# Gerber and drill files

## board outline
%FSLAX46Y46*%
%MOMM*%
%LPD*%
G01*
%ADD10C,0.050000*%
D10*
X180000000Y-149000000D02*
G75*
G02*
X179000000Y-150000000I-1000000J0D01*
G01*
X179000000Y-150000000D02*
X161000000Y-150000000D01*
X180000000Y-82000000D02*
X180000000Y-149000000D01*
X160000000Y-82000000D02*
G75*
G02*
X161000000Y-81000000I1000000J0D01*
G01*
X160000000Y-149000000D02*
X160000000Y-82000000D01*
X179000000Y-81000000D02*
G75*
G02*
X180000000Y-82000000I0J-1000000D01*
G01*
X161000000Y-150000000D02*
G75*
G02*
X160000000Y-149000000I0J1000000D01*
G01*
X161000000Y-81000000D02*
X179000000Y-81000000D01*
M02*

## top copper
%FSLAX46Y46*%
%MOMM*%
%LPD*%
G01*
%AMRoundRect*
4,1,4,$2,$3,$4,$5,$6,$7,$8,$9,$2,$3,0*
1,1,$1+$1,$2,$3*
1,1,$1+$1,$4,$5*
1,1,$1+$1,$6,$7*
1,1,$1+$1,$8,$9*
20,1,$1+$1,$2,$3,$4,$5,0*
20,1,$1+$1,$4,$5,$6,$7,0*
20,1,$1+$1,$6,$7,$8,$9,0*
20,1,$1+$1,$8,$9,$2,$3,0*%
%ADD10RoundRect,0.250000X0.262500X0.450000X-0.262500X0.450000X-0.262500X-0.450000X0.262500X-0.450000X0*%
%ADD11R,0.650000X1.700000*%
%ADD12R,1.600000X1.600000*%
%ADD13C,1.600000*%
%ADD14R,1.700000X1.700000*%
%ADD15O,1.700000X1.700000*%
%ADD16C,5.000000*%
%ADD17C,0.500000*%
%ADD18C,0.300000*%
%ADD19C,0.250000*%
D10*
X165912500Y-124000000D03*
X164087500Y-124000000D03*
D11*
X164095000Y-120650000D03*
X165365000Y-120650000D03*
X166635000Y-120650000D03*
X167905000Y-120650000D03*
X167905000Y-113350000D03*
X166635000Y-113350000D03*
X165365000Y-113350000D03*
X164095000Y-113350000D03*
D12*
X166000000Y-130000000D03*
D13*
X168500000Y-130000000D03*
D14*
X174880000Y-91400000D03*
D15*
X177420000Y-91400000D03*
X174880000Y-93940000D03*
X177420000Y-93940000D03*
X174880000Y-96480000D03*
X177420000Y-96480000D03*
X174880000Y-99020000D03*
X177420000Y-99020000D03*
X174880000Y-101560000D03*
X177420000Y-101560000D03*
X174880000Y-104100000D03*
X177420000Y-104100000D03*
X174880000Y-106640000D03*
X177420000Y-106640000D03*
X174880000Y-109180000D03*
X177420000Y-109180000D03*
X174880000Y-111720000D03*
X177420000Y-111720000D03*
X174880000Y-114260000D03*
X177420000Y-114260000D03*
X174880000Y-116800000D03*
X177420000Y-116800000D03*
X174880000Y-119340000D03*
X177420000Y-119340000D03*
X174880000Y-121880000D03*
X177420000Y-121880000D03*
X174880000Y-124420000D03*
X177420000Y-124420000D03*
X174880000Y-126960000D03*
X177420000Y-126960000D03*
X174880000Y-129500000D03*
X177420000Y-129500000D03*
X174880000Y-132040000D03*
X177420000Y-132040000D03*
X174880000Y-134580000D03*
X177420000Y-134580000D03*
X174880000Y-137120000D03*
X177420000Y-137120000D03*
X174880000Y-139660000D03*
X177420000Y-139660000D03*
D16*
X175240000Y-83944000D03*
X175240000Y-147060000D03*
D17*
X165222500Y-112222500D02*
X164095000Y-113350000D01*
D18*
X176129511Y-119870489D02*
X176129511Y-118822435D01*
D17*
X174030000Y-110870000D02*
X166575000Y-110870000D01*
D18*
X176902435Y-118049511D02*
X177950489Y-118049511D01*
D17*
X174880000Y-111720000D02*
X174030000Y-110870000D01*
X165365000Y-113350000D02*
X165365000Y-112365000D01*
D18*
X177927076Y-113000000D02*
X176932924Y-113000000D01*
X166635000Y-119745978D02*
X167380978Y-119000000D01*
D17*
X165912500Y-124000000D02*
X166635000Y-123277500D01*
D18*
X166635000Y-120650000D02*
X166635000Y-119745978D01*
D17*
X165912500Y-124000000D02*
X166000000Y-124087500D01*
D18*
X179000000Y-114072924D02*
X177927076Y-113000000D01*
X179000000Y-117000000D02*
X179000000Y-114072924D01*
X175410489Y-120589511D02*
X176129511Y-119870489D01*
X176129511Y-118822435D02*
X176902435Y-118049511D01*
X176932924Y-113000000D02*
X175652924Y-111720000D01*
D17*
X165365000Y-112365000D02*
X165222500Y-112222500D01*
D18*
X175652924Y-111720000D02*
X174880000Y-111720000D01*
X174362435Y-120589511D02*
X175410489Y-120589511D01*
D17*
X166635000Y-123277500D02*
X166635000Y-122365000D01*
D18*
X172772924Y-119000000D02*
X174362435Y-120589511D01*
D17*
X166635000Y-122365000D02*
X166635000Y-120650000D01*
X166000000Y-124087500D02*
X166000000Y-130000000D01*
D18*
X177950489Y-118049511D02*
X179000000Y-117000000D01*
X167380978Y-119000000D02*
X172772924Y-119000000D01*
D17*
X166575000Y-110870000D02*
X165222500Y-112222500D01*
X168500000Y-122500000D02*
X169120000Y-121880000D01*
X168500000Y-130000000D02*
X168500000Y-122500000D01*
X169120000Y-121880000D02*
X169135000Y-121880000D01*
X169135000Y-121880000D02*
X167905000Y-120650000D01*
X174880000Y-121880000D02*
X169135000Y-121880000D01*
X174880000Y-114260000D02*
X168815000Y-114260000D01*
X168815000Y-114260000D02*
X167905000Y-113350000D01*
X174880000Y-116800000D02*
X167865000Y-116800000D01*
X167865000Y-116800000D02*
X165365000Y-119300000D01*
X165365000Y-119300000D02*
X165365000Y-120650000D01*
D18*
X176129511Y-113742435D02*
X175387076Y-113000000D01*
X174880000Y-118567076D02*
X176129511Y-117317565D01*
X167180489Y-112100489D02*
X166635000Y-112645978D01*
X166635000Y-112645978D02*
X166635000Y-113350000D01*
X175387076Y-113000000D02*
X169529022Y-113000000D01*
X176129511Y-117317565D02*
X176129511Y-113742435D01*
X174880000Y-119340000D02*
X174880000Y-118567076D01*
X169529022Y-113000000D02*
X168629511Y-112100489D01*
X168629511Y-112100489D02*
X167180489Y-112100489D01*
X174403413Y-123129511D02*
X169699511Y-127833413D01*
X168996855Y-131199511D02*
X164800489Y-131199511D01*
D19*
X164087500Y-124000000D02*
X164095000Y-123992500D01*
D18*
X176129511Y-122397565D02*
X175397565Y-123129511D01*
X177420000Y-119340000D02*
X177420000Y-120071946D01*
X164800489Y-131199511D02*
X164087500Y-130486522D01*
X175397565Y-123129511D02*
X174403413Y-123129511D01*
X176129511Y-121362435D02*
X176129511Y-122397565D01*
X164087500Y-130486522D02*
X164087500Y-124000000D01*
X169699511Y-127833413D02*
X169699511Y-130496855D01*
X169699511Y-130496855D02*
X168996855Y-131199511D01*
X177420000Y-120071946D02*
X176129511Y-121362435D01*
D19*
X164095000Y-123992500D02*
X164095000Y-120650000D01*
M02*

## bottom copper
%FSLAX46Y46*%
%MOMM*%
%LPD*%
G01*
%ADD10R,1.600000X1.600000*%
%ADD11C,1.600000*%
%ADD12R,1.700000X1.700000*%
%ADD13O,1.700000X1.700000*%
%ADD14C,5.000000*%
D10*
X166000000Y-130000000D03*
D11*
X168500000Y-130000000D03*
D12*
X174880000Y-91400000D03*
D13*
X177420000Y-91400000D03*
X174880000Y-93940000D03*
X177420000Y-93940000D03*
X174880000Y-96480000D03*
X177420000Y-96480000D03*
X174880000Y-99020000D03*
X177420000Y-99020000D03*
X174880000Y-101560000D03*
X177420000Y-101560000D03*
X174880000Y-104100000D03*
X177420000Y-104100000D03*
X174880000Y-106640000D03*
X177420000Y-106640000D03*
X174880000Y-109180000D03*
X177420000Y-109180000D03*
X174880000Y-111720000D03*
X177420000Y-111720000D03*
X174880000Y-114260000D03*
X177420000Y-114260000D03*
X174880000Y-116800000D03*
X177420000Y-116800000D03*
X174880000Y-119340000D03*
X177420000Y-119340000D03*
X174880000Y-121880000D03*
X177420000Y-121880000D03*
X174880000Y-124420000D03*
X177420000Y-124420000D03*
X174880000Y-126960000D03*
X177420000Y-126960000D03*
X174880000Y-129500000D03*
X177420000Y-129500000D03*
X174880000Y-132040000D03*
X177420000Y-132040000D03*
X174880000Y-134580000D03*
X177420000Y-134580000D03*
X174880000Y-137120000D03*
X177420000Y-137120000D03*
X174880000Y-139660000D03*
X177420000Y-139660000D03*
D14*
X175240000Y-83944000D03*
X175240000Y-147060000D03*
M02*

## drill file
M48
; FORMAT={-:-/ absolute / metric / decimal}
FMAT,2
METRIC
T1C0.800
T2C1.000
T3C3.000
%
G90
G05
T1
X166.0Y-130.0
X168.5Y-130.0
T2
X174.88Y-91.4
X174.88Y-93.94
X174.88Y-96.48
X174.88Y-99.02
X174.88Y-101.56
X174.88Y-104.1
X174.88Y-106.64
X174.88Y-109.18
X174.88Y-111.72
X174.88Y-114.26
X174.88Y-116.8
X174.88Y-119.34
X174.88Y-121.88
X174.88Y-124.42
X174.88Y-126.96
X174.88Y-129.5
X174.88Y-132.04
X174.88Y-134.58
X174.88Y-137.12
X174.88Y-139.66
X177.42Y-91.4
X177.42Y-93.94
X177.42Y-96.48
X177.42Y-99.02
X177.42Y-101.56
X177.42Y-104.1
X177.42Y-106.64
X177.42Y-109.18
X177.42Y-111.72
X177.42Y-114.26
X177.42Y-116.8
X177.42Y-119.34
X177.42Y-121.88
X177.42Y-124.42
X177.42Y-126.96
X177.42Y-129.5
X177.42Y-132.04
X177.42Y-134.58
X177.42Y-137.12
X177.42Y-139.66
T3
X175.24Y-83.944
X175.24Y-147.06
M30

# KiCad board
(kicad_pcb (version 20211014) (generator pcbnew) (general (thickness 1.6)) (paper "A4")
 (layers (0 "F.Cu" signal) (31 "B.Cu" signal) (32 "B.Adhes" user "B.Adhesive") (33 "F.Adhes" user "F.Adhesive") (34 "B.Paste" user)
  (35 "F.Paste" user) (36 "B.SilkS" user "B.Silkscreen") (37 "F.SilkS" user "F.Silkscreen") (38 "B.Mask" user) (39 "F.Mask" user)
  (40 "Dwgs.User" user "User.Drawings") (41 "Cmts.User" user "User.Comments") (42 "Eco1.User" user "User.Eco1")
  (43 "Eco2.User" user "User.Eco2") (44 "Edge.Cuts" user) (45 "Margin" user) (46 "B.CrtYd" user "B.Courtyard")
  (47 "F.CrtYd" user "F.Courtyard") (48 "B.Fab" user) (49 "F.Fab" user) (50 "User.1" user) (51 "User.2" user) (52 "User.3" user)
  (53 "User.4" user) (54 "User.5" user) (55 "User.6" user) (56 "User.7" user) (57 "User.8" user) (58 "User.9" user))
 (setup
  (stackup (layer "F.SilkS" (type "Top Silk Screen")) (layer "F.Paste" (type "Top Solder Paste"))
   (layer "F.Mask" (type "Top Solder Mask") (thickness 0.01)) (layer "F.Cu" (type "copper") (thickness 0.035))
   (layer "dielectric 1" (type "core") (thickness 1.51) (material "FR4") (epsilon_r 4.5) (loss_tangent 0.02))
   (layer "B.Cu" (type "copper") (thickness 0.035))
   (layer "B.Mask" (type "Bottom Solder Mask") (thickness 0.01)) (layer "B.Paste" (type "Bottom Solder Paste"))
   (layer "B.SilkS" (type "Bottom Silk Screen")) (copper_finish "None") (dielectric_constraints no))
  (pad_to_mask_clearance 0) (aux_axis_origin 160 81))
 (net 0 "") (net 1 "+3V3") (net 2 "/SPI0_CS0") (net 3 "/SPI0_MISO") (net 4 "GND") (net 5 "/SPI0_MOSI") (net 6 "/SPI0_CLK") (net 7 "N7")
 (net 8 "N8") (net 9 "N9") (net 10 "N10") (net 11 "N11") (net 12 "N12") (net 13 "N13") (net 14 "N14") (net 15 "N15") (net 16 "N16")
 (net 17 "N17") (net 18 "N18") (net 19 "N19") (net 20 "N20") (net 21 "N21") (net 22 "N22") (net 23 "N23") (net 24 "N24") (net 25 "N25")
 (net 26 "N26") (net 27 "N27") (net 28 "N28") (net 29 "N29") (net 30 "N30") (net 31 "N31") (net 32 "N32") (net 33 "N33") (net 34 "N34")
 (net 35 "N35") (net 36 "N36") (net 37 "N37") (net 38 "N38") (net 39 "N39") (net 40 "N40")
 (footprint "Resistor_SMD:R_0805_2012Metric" (layer "F.Cu") (at 165 124 180)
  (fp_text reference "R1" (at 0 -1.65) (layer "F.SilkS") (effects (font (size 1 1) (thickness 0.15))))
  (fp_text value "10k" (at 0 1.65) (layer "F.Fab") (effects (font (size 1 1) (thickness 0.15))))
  (pad "1" smd roundrect (at -0.9125 0 180) (size 1.025 1.4) (layers "F.Cu" "F.Paste" "F.Mask") (roundrect_rratio 0.243902439)
   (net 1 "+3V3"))
  (pad "2" smd roundrect (at 0.9125 0 180) (size 1.025 1.4) (layers "F.Cu" "F.Paste" "F.Mask") (roundrect_rratio 0.243902439)
   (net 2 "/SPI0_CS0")))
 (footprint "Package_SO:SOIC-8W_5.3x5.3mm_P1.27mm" (layer "F.Cu") (at 166 117 90)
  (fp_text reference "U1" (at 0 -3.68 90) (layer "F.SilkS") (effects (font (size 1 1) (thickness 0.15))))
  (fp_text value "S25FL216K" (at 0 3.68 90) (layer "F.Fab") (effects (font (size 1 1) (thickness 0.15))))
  (pad "1" smd rect (at -3.65 -1.905 90) (size 1.7 0.65) (layers "F.Cu" "F.Paste" "F.Mask") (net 2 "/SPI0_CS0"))
  (pad "2" smd rect (at -3.65 -0.635 90) (size 1.7 0.65) (layers "F.Cu" "F.Paste" "F.Mask") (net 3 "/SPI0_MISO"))
  (pad "3" smd rect (at -3.65 0.635 90) (size 1.7 0.65) (layers "F.Cu" "F.Paste" "F.Mask") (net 1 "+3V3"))
  (pad "4" smd rect (at -3.65 1.905 90) (size 1.7 0.65) (layers "F.Cu" "F.Paste" "F.Mask") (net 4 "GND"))
  (pad "5" smd rect (at 3.65 1.905 90) (size 1.7 0.65) (layers "F.Cu" "F.Paste" "F.Mask") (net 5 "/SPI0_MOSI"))
  (pad "6" smd rect (at 3.65 0.635 90) (size 1.7 0.65) (layers "F.Cu" "F.Paste" "F.Mask") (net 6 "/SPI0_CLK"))
  (pad "7" smd rect (at 3.65 -0.635 90) (size 1.7 0.65) (layers "F.Cu" "F.Paste" "F.Mask") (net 1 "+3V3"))
  (pad "8" smd rect (at 3.65 -1.905 90) (size 1.7 0.65) (layers "F.Cu" "F.Paste" "F.Mask") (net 1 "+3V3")))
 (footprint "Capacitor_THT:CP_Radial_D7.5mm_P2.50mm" (layer "F.Cu") (at 166 130)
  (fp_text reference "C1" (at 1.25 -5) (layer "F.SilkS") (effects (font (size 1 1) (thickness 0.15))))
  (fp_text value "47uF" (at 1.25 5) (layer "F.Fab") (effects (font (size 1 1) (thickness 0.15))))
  (pad "1" thru_hole rect (at 0 0) (size 1.6 1.6) (drill 0.8) (layers *.Cu *.Mask) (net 1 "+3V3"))
  (pad "2" thru_hole circle (at 2.5 0) (size 1.6 1.6) (drill 0.8) (layers *.Cu *.Mask) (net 4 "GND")))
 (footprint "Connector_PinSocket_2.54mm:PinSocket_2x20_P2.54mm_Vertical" (layer "B.Cu") (at 174.88 91.4 180)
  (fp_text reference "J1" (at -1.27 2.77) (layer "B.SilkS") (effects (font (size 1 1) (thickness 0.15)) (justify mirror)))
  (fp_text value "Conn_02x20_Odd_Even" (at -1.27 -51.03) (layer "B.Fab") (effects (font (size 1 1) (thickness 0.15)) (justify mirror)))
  (pad "1" thru_hole rect (at 0 0 180) (size 1.7 1.7) (drill 1) (layers *.Cu *.Mask) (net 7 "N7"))
  (pad "2" thru_hole oval (at -2.54 0 180) (size 1.7 1.7) (drill 1) (layers *.Cu *.Mask) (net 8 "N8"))
  (pad "3" thru_hole oval (at 0 -2.54 180) (size 1.7 1.7) (drill 1) (layers *.Cu *.Mask) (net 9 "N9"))
  (pad "4" thru_hole oval (at -2.54 -2.54 180) (size 1.7 1.7) (drill 1) (layers *.Cu *.Mask) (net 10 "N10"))
  (pad "5" thru_hole oval (at 0 -5.08 180) (size 1.7 1.7) (drill 1) (layers *.Cu *.Mask) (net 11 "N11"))
  (pad "6" thru_hole oval (at -2.54 -5.08 180) (size 1.7 1.7) (drill 1) (layers *.Cu *.Mask) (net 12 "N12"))
  (pad "7" thru_hole oval (at 0 -7.62 180) (size 1.7 1.7) (drill 1) (layers *.Cu *.Mask) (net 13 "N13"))
  (pad "8" thru_hole oval (at -2.54 -7.62 180) (size 1.7 1.7) (drill 1) (layers *.Cu *.Mask) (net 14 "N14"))
  (pad "9" thru_hole oval (at 0 -10.16 180) (size 1.7 1.7) (drill 1) (layers *.Cu *.Mask) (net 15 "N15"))
  (pad "10" thru_hole oval (at -2.54 -10.16 180) (size 1.7 1.7) (drill 1) (layers *.Cu *.Mask) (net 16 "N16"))
  (pad "11" thru_hole oval (at 0 -12.7 180) (size 1.7 1.7) (drill 1) (layers *.Cu *.Mask) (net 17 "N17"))
  (pad "12" thru_hole oval (at -2.54 -12.7 180) (size 1.7 1.7) (drill 1) (layers *.Cu *.Mask) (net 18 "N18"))
  (pad "13" thru_hole oval (at 0 -15.24 180) (size 1.7 1.7) (drill 1) (layers *.Cu *.Mask) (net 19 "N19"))
  (pad "14" thru_hole oval (at -2.54 -15.24 180) (size 1.7 1.7) (drill 1) (layers *.Cu *.Mask) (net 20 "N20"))
  (pad "15" thru_hole oval (at 0 -17.78 180) (size 1.7 1.7) (drill 1) (layers *.Cu *.Mask) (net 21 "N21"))
  (pad "16" thru_hole oval (at -2.54 -17.78 180) (size 1.7 1.7) (drill 1) (layers *.Cu *.Mask) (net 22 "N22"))
  (pad "17" thru_hole oval (at 0 -20.32 180) (size 1.7 1.7) (drill 1) (layers *.Cu *.Mask) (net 1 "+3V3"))
  (pad "18" thru_hole oval (at -2.54 -20.32 180) (size 1.7 1.7) (drill 1) (layers *.Cu *.Mask) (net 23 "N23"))
  (pad "19" thru_hole oval (at 0 -22.86 180) (size 1.7 1.7) (drill 1) (layers *.Cu *.Mask) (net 5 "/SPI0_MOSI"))
  (pad "20" thru_hole oval (at -2.54 -22.86 180) (size 1.7 1.7) (drill 1) (layers *.Cu *.Mask) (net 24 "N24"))
  (pad "21" thru_hole oval (at 0 -25.4 180) (size 1.7 1.7) (drill 1) (layers *.Cu *.Mask) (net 3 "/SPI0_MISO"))
  (pad "22" thru_hole oval (at -2.54 -25.4 180) (size 1.7 1.7) (drill 1) (layers *.Cu *.Mask) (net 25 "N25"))
  (pad "23" thru_hole oval (at 0 -27.94 180) (size 1.7 1.7) (drill 1) (layers *.Cu *.Mask) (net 6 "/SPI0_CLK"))
  (pad "24" thru_hole oval (at -2.54 -27.94 180) (size 1.7 1.7) (drill 1) (layers *.Cu *.Mask) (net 2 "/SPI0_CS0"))
  (pad "25" thru_hole oval (at 0 -30.48 180) (size 1.7 1.7) (drill 1) (layers *.Cu *.Mask) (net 4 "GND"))
  (pad "26" thru_hole oval (at -2.54 -30.48 180) (size 1.7 1.7) (drill 1) (layers *.Cu *.Mask) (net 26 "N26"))
  (pad "27" thru_hole oval (at 0 -33.02 180) (size 1.7 1.7) (drill 1) (layers *.Cu *.Mask) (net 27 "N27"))
  (pad "28" thru_hole oval (at -2.54 -33.02 180) (size 1.7 1.7) (drill 1) (layers *.Cu *.Mask) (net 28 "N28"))
  (pad "29" thru_hole oval (at 0 -35.56 180) (size 1.7 1.7) (drill 1) (layers *.Cu *.Mask) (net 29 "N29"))
  (pad "30" thru_hole oval (at -2.54 -35.56 180) (size 1.7 1.7) (drill 1) (layers *.Cu *.Mask) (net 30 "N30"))
  (pad "31" thru_hole oval (at 0 -38.1 180) (size 1.7 1.7) (drill 1) (layers *.Cu *.Mask) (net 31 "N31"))
  (pad "32" thru_hole oval (at -2.54 -38.1 180) (size 1.7 1.7) (drill 1) (layers *.Cu *.Mask) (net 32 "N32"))
  (pad "33" thru_hole oval (at 0 -40.64 180) (size 1.7 1.7) (drill 1) (layers *.Cu *.Mask) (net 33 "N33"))
  (pad "34" thru_hole oval (at -2.54 -40.64 180) (size 1.7 1.7) (drill 1) (layers *.Cu *.Mask) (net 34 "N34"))
  (pad "35" thru_hole oval (at 0 -43.18 180) (size 1.7 1.7) (drill 1) (layers *.Cu *.Mask) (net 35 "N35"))
  (pad "36" thru_hole oval (at -2.54 -43.18 180) (size 1.7 1.7) (drill 1) (layers *.Cu *.Mask) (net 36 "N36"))
  (pad "37" thru_hole oval (at 0 -45.72 180) (size 1.7 1.7) (drill 1) (layers *.Cu *.Mask) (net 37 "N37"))
  (pad "38" thru_hole oval (at -2.54 -45.72 180) (size 1.7 1.7) (drill 1) (layers *.Cu *.Mask) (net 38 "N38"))
  (pad "39" thru_hole oval (at 0 -48.26 180) (size 1.7 1.7) (drill 1) (layers *.Cu *.Mask) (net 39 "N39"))
  (pad "40" thru_hole oval (at -2.54 -48.26 180) (size 1.7 1.7) (drill 1) (layers *.Cu *.Mask) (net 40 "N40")))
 (gr_arc (start 180 149) (mid 179.707107 149.707107) (end 179 150) (layer "Edge.Cuts") (width 0.05))
 (gr_line (start 179 150) (end 161 150) (layer "Edge.Cuts") (width 0.05))
 (gr_line (start 180 82) (end 180 149) (layer "Edge.Cuts") (width 0.05))
 (gr_arc (start 160 82) (mid 160.292893 81.292893) (end 161 81) (layer "Edge.Cuts") (width 0.05))
 (gr_line (start 160 149) (end 160 82) (layer "Edge.Cuts") (width 0.05))
 (gr_arc (start 179 81) (mid 179.707107 81.292893) (end 180 82) (layer "Edge.Cuts") (width 0.05))
 (gr_arc (start 161 150) (mid 160.292893 149.707107) (end 160 149) (layer "Edge.Cuts") (width 0.05))
 (gr_line (start 161 81) (end 179 81) (layer "Edge.Cuts") (width 0.05))
 (via (at 175.24 83.944) (size 5) (drill 3) (layers "F.Cu" "B.Cu") (free) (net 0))
 (via (at 175.24 147.06) (size 5) (drill 3) (layers "F.Cu" "B.Cu") (free) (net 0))
 (segment (start 165.2225 112.2225) (end 164.095 113.35) (width 0.5) (layer "F.Cu") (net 1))
 (segment (start 176.129511 119.870489) (end 176.129511 118.822435) (width 0.3) (layer "F.Cu") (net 1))
 (segment (start 174.03 110.87) (end 166.575 110.87) (width 0.5) (layer "F.Cu") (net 1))
 (segment (start 176.902435 118.049511) (end 177.950489 118.049511) (width 0.3) (layer "F.Cu") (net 1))
 (segment (start 174.88 111.72) (end 174.03 110.87) (width 0.5) (layer "F.Cu") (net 1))
 (segment (start 165.365 113.35) (end 165.365 112.365) (width 0.5) (layer "F.Cu") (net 1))
 (segment (start 177.927076 113) (end 176.932924 113) (width 0.3) (layer "F.Cu") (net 1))
 (segment (start 166.635 119.745978) (end 167.380978 119) (width 0.3) (layer "F.Cu") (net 1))
 (segment (start 165.9125 124) (end 166.635 123.2775) (width 0.5) (layer "F.Cu") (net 1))
 (segment (start 166.635 120.65) (end 166.635 119.745978) (width 0.3) (layer "F.Cu") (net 1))
 (segment (start 165.9125 124) (end 166 124.0875) (width 0.5) (layer "F.Cu") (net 1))
 (segment (start 179 114.072924) (end 177.927076 113) (width 0.3) (layer "F.Cu") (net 1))
 (segment (start 179 117) (end 179 114.072924) (width 0.3) (layer "F.Cu") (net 1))
 (segment (start 175.410489 120.589511) (end 176.129511 119.870489) (width 0.3) (layer "F.Cu") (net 1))
 (segment (start 176.129511 118.822435) (end 176.902435 118.049511) (width 0.3) (layer "F.Cu") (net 1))
 (segment (start 176.932924 113) (end 175.652924 111.72) (width 0.3) (layer "F.Cu") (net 1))
 (segment (start 165.365 112.365) (end 165.2225 112.2225) (width 0.5) (layer "F.Cu") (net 1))
 (segment (start 175.652924 111.72) (end 174.88 111.72) (width 0.3) (layer "F.Cu") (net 1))
 (segment (start 174.362435 120.589511) (end 175.410489 120.589511) (width 0.3) (layer "F.Cu") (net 1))
 (segment (start 166.635 123.2775) (end 166.635 122.365) (width 0.5) (layer "F.Cu") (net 1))
 (segment (start 172.772924 119) (end 174.362435 120.589511) (width 0.3) (layer "F.Cu") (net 1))
 (segment (start 166.635 122.365) (end 166.635 120.65) (width 0.5) (layer "F.Cu") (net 1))
 (segment (start 166 124.0875) (end 166 130) (width 0.5) (layer "F.Cu") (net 1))
 (segment (start 177.950489 118.049511) (end 179 117) (width 0.3) (layer "F.Cu") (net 1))
 (segment (start 167.380978 119) (end 172.772924 119) (width 0.3) (layer "F.Cu") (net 1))
 (segment (start 166.575 110.87) (end 165.2225 112.2225) (width 0.5) (layer "F.Cu") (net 1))
 (segment (start 168.5 122.5) (end 169.12 121.88) (width 0.5) (layer "F.Cu") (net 4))
 (segment (start 168.5 130) (end 168.5 122.5) (width 0.5) (layer "F.Cu") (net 4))
 (segment (start 169.12 121.88) (end 169.135 121.88) (width 0.5) (layer "F.Cu") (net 4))
 (segment (start 169.135 121.88) (end 167.905 120.65) (width 0.5) (layer "F.Cu") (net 4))
 (segment (start 174.88 121.88) (end 169.135 121.88) (width 0.5) (layer "F.Cu") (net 4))
 (segment (start 174.88 114.26) (end 168.815 114.26) (width 0.5) (layer "F.Cu") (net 5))
 (segment (start 168.815 114.26) (end 167.905 113.35) (width 0.5) (layer "F.Cu") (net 5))
 (segment (start 174.88 116.8) (end 167.865 116.8) (width 0.5) (layer "F.Cu") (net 3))
 (segment (start 167.865 116.8) (end 165.365 119.3) (width 0.5) (layer "F.Cu") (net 3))
 (segment (start 165.365 119.3) (end 165.365 120.65) (width 0.5) (layer "F.Cu") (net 3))
 (segment (start 176.129511 113.742435) (end 175.387076 113) (width 0.3) (layer "F.Cu") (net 6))
 (segment (start 174.88 118.567076) (end 176.129511 117.317565) (width 0.3) (layer "F.Cu") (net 6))
 (segment (start 167.180489 112.100489) (end 166.635 112.645978) (width 0.3) (layer "F.Cu") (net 6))
 (segment (start 166.635 112.645978) (end 166.635 113.35) (width 0.3) (layer "F.Cu") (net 6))
 (segment (start 175.387076 113) (end 169.529022 113) (width 0.3) (layer "F.Cu") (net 6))
 (segment (start 176.129511 117.317565) (end 176.129511 113.742435) (width 0.3) (layer "F.Cu") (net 6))
 (segment (start 174.88 119.34) (end 174.88 118.567076) (width 0.3) (layer "F.Cu") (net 6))
 (segment (start 169.529022 113) (end 168.629511 112.100489) (width 0.3) (layer "F.Cu") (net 6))
 (segment (start 168.629511 112.100489) (end 167.180489 112.100489) (width 0.3) (layer "F.Cu") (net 6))
 (segment (start 174.403413 123.129511) (end 169.699511 127.833413) (width 0.3) (layer "F.Cu") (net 2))
 (segment (start 168.996855 131.199511) (end 164.800489 131.199511) (width 0.3) (layer "F.Cu") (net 2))
 (segment (start 164.0875 124) (end 164.095 123.9925) (width 0.25) (layer "F.Cu") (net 2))
 (segment (start 176.129511 122.397565) (end 175.397565 123.129511) (width 0.3) (layer "F.Cu") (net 2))
 (segment (start 177.42 119.34) (end 177.42 120.071946) (width 0.3) (layer "F.Cu") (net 2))
 (segment (start 164.800489 131.199511) (end 164.0875 130.486522) (width 0.3) (layer "F.Cu") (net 2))
 (segment (start 175.397565 123.129511) (end 174.403413 123.129511) (width 0.3) (layer "F.Cu") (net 2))
 (segment (start 176.129511 121.362435) (end 176.129511 122.397565) (width 0.3) (layer "F.Cu") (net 2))
 (segment (start 164.0875 130.486522) (end 164.0875 124) (width 0.3) (layer "F.Cu") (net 2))
 (segment (start 169.699511 127.833413) (end 169.699511 130.496855) (width 0.3) (layer "F.Cu") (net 2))
 (segment (start 169.699511 130.496855) (end 168.996855 131.199511) (width 0.3) (layer "F.Cu") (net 2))
 (segment (start 177.42 120.071946) (end 176.129511 121.362435) (width 0.3) (layer "F.Cu") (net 2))
 (segment (start 164.095 123.9925) (end 164.095 120.65) (width 0.25) (layer "F.Cu") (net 2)))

